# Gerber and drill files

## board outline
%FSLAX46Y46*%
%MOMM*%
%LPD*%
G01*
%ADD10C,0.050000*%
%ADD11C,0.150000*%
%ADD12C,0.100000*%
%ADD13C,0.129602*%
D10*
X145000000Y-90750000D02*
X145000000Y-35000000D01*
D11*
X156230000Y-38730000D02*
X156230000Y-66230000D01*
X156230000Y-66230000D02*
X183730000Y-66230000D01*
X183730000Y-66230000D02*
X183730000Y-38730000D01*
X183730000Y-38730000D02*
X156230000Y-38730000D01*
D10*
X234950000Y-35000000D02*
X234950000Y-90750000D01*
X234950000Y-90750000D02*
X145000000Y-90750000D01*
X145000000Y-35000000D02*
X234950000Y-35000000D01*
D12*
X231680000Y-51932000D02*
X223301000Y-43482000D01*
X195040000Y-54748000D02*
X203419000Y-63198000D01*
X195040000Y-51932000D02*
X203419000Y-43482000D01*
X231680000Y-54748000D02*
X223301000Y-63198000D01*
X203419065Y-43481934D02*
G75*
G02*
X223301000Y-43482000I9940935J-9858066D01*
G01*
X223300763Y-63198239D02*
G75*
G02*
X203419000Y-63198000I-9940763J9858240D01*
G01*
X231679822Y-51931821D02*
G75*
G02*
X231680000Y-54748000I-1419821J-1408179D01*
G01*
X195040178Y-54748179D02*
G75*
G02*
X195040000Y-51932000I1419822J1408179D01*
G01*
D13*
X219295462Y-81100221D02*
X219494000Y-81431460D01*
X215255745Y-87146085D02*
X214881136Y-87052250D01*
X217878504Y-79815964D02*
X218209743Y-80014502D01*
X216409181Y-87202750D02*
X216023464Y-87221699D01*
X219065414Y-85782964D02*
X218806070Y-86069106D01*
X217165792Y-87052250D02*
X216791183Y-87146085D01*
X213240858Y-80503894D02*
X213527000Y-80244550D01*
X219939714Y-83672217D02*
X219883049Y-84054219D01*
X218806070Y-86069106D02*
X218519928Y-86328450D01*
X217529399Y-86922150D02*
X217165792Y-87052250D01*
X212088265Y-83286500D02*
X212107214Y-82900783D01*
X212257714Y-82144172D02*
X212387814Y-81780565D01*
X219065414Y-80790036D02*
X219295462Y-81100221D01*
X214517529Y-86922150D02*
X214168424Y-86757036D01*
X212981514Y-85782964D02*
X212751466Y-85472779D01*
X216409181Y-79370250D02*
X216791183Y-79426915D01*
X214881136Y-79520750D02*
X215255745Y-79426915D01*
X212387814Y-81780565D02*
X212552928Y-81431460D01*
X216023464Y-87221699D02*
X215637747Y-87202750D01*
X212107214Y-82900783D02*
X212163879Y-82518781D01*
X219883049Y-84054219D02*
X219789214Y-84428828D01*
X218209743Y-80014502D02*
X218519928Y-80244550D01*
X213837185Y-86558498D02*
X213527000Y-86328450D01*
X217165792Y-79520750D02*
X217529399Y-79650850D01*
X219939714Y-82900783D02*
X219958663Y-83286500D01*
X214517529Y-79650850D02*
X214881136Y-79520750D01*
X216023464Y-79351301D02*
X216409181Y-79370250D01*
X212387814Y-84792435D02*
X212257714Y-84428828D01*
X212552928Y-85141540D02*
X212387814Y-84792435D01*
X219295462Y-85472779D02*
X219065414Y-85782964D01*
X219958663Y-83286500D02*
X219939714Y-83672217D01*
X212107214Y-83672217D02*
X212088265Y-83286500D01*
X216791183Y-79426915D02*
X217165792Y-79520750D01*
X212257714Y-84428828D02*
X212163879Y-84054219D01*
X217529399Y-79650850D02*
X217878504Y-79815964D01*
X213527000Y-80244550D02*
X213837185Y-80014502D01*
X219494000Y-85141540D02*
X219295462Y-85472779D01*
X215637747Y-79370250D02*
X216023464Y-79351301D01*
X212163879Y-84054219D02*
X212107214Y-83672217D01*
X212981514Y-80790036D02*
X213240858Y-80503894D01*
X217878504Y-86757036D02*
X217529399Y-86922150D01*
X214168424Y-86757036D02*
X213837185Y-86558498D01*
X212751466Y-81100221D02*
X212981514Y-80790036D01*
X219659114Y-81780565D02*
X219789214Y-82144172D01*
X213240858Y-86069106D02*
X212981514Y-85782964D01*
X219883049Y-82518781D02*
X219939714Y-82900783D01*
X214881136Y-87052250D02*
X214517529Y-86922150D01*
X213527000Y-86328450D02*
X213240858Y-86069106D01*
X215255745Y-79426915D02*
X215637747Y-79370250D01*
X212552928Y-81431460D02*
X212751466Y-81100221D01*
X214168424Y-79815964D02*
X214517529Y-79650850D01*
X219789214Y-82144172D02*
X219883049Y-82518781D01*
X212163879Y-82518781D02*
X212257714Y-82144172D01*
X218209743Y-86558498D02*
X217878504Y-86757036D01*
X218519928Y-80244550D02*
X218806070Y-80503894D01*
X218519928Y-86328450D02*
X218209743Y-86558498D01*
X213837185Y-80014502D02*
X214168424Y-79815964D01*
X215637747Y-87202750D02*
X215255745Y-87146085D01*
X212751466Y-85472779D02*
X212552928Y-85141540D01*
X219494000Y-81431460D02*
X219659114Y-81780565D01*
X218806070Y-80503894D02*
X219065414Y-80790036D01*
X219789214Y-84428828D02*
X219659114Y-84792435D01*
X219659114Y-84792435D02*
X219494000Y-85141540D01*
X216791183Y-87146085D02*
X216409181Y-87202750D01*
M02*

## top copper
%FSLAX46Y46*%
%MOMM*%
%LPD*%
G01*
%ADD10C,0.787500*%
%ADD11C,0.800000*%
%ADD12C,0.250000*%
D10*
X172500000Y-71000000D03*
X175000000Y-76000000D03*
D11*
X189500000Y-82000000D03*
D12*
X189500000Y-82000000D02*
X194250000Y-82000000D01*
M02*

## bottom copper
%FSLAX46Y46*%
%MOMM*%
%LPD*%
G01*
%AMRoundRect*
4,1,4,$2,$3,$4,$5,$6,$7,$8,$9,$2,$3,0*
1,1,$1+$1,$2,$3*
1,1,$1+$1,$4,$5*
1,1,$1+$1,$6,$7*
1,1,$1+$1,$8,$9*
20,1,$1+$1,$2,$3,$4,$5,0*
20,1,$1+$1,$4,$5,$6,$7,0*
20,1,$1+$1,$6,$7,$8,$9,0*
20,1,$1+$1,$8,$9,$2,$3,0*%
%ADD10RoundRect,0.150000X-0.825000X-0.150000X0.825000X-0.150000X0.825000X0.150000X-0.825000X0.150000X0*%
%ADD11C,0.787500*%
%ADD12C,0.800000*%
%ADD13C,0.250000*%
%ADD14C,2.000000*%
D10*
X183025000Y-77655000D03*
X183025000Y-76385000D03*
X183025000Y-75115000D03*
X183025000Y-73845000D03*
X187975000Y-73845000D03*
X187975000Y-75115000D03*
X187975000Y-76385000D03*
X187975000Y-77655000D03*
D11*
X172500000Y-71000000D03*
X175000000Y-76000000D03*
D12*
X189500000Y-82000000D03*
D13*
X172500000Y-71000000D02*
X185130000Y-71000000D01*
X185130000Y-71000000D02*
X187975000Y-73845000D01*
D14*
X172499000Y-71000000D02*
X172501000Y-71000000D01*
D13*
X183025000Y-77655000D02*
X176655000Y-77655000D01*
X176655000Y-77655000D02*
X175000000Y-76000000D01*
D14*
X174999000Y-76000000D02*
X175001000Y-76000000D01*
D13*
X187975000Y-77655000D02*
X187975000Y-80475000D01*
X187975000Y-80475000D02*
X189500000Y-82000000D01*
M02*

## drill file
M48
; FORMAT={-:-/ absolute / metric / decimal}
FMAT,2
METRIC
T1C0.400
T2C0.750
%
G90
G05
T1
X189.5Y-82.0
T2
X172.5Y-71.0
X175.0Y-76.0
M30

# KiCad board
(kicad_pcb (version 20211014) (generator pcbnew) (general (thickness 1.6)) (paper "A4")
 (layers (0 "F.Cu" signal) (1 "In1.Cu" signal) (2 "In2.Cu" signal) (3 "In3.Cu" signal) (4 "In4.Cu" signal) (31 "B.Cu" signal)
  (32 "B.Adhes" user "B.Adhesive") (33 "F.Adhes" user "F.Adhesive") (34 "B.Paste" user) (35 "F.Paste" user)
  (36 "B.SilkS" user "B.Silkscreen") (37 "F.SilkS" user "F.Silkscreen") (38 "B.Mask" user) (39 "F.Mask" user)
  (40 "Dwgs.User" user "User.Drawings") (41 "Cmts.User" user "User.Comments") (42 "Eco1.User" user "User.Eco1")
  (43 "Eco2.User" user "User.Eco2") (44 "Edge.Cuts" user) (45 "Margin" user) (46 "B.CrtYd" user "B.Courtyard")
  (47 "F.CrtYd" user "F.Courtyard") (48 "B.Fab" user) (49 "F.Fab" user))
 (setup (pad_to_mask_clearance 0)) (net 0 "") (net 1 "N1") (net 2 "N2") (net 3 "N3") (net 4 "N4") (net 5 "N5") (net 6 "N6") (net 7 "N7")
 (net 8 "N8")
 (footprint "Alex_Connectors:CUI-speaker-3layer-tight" (layer "F.Cu") (at 213.36 53.34 180)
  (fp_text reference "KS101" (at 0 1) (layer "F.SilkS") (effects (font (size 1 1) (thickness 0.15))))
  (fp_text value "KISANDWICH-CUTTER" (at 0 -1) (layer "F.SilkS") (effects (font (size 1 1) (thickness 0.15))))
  (fp_line (start -18.32 1.408) (end -9.941 9.858) (layer "Edge.Cuts") (width 0.1))
  (fp_line (start 18.32 -1.408) (end 9.941 -9.858) (layer "Edge.Cuts") (width 0.1))
  (fp_line (start 18.32 1.408) (end 9.941 9.858) (layer "Edge.Cuts") (width 0.1))
  (fp_line (start -18.32 -1.408) (end -9.941 -9.858) (layer "Edge.Cuts") (width 0.1))
  (fp_arc (start 9.940935 9.858066) (mid -0.000046 14.00013) (end -9.941 9.858) (layer "Edge.Cuts") (width 0.1))
  (fp_arc (start -9.940763 -9.858239) (mid 0.000168 -14.00013) (end 9.941 -9.858) (layer "Edge.Cuts") (width 0.1))
  (fp_arc (start -18.319822 1.408179) (mid -18.899716 0.000126) (end -18.32 -1.408) (layer "Edge.Cuts") (width 0.1))
  (fp_arc (start 18.319822 -1.408179) (mid 18.899716 -0.000126) (end 18.32 1.408) (layer "Edge.Cuts") (width 0.1)))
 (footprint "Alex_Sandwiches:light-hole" (layer "F.Cu") (at 201.93 77.47)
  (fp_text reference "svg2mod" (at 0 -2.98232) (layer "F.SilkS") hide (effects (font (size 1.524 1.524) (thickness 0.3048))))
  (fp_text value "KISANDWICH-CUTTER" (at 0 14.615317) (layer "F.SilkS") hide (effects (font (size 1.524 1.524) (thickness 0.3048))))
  (fp_line (start 17.365462 3.630221) (end 17.564 3.96146) (layer "Edge.Cuts") (width 0.129602))
  (fp_line (start 13.325745 9.676085) (end 12.951136 9.58225) (layer "Edge.Cuts") (width 0.129602))
  (fp_line (start 15.948504 2.345964) (end 16.279743 2.544502) (layer "Edge.Cuts") (width 0.129602))
  (fp_line (start 14.479181 9.73275) (end 14.093464 9.751699) (layer "Edge.Cuts") (width 0.129602))
  (fp_line (start 17.135414 8.312964) (end 16.87607 8.599106) (layer "Edge.Cuts") (width 0.129602))
  (fp_line (start 15.235792 9.58225) (end 14.861183 9.676085) (layer "Edge.Cuts") (width 0.129602))
  (fp_line (start 11.310858 3.033894) (end 11.597 2.77455) (layer "Edge.Cuts") (width 0.129602))
  (fp_line (start 18.009714 6.202217) (end 17.953049 6.584219) (layer "Edge.Cuts") (width 0.129602))
  (fp_line (start 16.87607 8.599106) (end 16.589928 8.85845) (layer "Edge.Cuts") (width 0.129602))
  (fp_line (start 15.599399 9.45215) (end 15.235792 9.58225) (layer "Edge.Cuts") (width 0.129602))
  (fp_line (start 10.158265 5.8165) (end 10.177214 5.430783) (layer "Edge.Cuts") (width 0.129602))
  (fp_line (start 10.327714 4.674172) (end 10.457814 4.310565) (layer "Edge.Cuts") (width 0.129602))
  (fp_line (start 17.135414 3.320036) (end 17.365462 3.630221) (layer "Edge.Cuts") (width 0.129602))
  (fp_line (start 12.587529 9.45215) (end 12.238424 9.287036) (layer "Edge.Cuts") (width 0.129602))
  (fp_line (start 11.051514 8.312964) (end 10.821466 8.002779) (layer "Edge.Cuts") (width 0.129602))
  (fp_line (start 14.479181 1.90025) (end 14.861183 1.956915) (layer "Edge.Cuts") (width 0.129602))
  (fp_line (start 12.951136 2.05075) (end 13.325745 1.956915) (layer "Edge.Cuts") (width 0.129602))
  (fp_line (start 10.457814 4.310565) (end 10.622928 3.96146) (layer "Edge.Cuts") (width 0.129602))
  (fp_line (start 14.093464 9.751699) (end 13.707747 9.73275) (layer "Edge.Cuts") (width 0.129602))
  (fp_line (start 10.177214 5.430783) (end 10.233879 5.048781) (layer "Edge.Cuts") (width 0.129602))
  (fp_line (start 17.953049 6.584219) (end 17.859214 6.958828) (layer "Edge.Cuts") (width 0.129602))
  (fp_line (start 16.279743 2.544502) (end 16.589928 2.77455) (layer "Edge.Cuts") (width 0.129602))
  (fp_line (start 11.907185 9.088498) (end 11.597 8.85845) (layer "Edge.Cuts") (width 0.129602))
  (fp_line (start 15.235792 2.05075) (end 15.599399 2.18085) (layer "Edge.Cuts") (width 0.129602))
  (fp_line (start 18.009714 5.430783) (end 18.028663 5.8165) (layer "Edge.Cuts") (width 0.129602))
  (fp_line (start 12.587529 2.18085) (end 12.951136 2.05075) (layer "Edge.Cuts") (width 0.129602))
  (fp_line (start 14.093464 1.881301) (end 14.479181 1.90025) (layer "Edge.Cuts") (width 0.129602))
  (fp_line (start 10.457814 7.322435) (end 10.327714 6.958828) (layer "Edge.Cuts") (width 0.129602))
  (fp_line (start 10.622928 7.67154) (end 10.457814 7.322435) (layer "Edge.Cuts") (width 0.129602))
  (fp_line (start 17.365462 8.002779) (end 17.135414 8.312964) (layer "Edge.Cuts") (width 0.129602))
  (fp_line (start 18.028663 5.8165) (end 18.009714 6.202217) (layer "Edge.Cuts") (width 0.129602))
  (fp_line (start 10.177214 6.202217) (end 10.158265 5.8165) (layer "Edge.Cuts") (width 0.129602))
  (fp_line (start 14.861183 1.956915) (end 15.235792 2.05075) (layer "Edge.Cuts") (width 0.129602))
  (fp_line (start 10.327714 6.958828) (end 10.233879 6.584219) (layer "Edge.Cuts") (width 0.129602))
  (fp_line (start 15.599399 2.18085) (end 15.948504 2.345964) (layer "Edge.Cuts") (width 0.129602))
  (fp_line (start 11.597 2.77455) (end 11.907185 2.544502) (layer "Edge.Cuts") (width 0.129602))
  (fp_line (start 17.564 7.67154) (end 17.365462 8.002779) (layer "Edge.Cuts") (width 0.129602))
  (fp_line (start 13.707747 1.90025) (end 14.093464 1.881301) (layer "Edge.Cuts") (width 0.129602))
  (fp_line (start 10.233879 6.584219) (end 10.177214 6.202217) (layer "Edge.Cuts") (width 0.129602))
  (fp_line (start 11.051514 3.320036) (end 11.310858 3.033894) (layer "Edge.Cuts") (width 0.129602))
  (fp_line (start 15.948504 9.287036) (end 15.599399 9.45215) (layer "Edge.Cuts") (width 0.129602))
  (fp_line (start 12.238424 9.287036) (end 11.907185 9.088498) (layer "Edge.Cuts") (width 0.129602))
  (fp_line (start 10.821466 3.630221) (end 11.051514 3.320036) (layer "Edge.Cuts") (width 0.129602))
  (fp_line (start 17.729114 4.310565) (end 17.859214 4.674172) (layer "Edge.Cuts") (width 0.129602))
  (fp_line (start 11.310858 8.599106) (end 11.051514 8.312964) (layer "Edge.Cuts") (width 0.129602))
  (fp_line (start 17.953049 5.048781) (end 18.009714 5.430783) (layer "Edge.Cuts") (width 0.129602))
  (fp_line (start 12.951136 9.58225) (end 12.587529 9.45215) (layer "Edge.Cuts") (width 0.129602))
  (fp_line (start 11.597 8.85845) (end 11.310858 8.599106) (layer "Edge.Cuts") (width 0.129602))
  (fp_line (start 13.325745 1.956915) (end 13.707747 1.90025) (layer "Edge.Cuts") (width 0.129602))
  (fp_line (start 10.622928 3.96146) (end 10.821466 3.630221) (layer "Edge.Cuts") (width 0.129602))
  (fp_line (start 12.238424 2.345964) (end 12.587529 2.18085) (layer "Edge.Cuts") (width 0.129602))
  (fp_line (start 17.859214 4.674172) (end 17.953049 5.048781) (layer "Edge.Cuts") (width 0.129602))
  (fp_line (start 10.233879 5.048781) (end 10.327714 4.674172) (layer "Edge.Cuts") (width 0.129602))
  (fp_line (start 16.279743 9.088498) (end 15.948504 9.287036) (layer "Edge.Cuts") (width 0.129602))
  (fp_line (start 16.589928 2.77455) (end 16.87607 3.033894) (layer "Edge.Cuts") (width 0.129602))
  (fp_line (start 16.589928 8.85845) (end 16.279743 9.088498) (layer "Edge.Cuts") (width 0.129602))
  (fp_line (start 11.907185 2.544502) (end 12.238424 2.345964) (layer "Edge.Cuts") (width 0.129602))
  (fp_line (start 13.707747 9.73275) (end 13.325745 9.676085) (layer "Edge.Cuts") (width 0.129602))
  (fp_line (start 10.821466 8.002779) (end 10.622928 7.67154) (layer "Edge.Cuts") (width 0.129602))
  (fp_line (start 17.564 3.96146) (end 17.729114 4.310565) (layer "Edge.Cuts") (width 0.129602))
  (fp_line (start 16.87607 3.033894) (end 17.135414 3.320036) (layer "Edge.Cuts") (width 0.129602))
  (fp_line (start 17.859214 6.958828) (end 17.729114 7.322435) (layer "Edge.Cuts") (width 0.129602))
  (fp_line (start 17.729114 7.322435) (end 17.564 7.67154) (layer "Edge.Cuts") (width 0.129602))
  (fp_line (start 14.861183 9.676085) (end 14.479181 9.73275) (layer "Edge.Cuts") (width 0.129602)))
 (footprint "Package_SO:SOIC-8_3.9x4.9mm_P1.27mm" (layer "B.Cu") (at 185.5 75.75)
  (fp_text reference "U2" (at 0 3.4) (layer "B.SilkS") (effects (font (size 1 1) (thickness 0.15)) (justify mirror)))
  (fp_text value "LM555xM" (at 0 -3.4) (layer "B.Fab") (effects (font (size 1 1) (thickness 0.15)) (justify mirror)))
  (pad "1" smd roundrect locked (at -2.475 1.905) (size 1.95 0.6) (layers "B.Cu" "B.Paste" "B.Mask") (roundrect_rratio 0.25) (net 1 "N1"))
  (pad "2" smd roundrect locked (at -2.475 0.635) (size 1.95 0.6) (layers "B.Cu" "B.Paste" "B.Mask") (roundrect_rratio 0.25) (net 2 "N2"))
  (pad "3" smd roundrect locked (at -2.475 -0.635) (size 1.95 0.6) (layers "B.Cu" "B.Paste" "B.Mask") (roundrect_rratio 0.25) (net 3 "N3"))
  (pad "4" smd roundrect locked (at -2.475 -1.905) (size 1.95 0.6) (layers "B.Cu" "B.Paste" "B.Mask") (roundrect_rratio 0.25) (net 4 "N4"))
  (pad "5" smd roundrect locked (at 2.475 -1.905) (size 1.95 0.6) (layers "B.Cu" "B.Paste" "B.Mask") (roundrect_rratio 0.25) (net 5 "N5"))
  (pad "6" smd roundrect locked (at 2.475 -0.635) (size 1.95 0.6) (layers "B.Cu" "B.Paste" "B.Mask") (roundrect_rratio 0.25) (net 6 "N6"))
  (pad "7" smd roundrect locked (at 2.475 0.635) (size 1.95 0.6) (layers "B.Cu" "B.Paste" "B.Mask") (roundrect_rratio 0.25) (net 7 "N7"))
  (pad "8" smd roundrect locked (at 2.475 1.905) (size 1.95 0.6) (layers "B.Cu" "B.Paste" "B.Mask") (roundrect_rratio 0.25) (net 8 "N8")))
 (gr_line (start 145 90.75) (end 145 35) (layer "Edge.Cuts") (width 0.05))
 (gr_line (start 156.23 38.73) (end 156.23 66.23) (layer "Edge.Cuts") (width 0.15))
 (gr_line (start 156.23 66.23) (end 183.73 66.23) (layer "Edge.Cuts") (width 0.15))
 (gr_line (start 183.73 66.23) (end 183.73 38.73) (layer "Edge.Cuts") (width 0.15))
 (gr_line (start 183.73 38.73) (end 156.23 38.73) (layer "Edge.Cuts") (width 0.15))
 (gr_line (start 234.95 35) (end 234.95 90.75) (layer "Edge.Cuts") (width 0.05))
 (gr_line (start 234.95 90.75) (end 145 90.75) (layer "Edge.Cuts") (width 0.05))
 (gr_line (start 145 35) (end 234.95 35) (layer "Edge.Cuts") (width 0.05))
 (via (at 172.5 71) (size 0.7875) (drill 0.75) (layers "F.Cu" "B.Cu") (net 5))
 (segment (start 172.5 71) (end 185.13 71) (width 0.25) (layer "B.Cu") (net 5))
 (segment (start 185.13 71) (end 187.975 73.845) (width 0.25) (layer "B.Cu") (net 5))
 (segment (start 172.499 71) (end 172.501 71) (width 2) (layer "B.Cu") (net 5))
 (via (at 175 76) (size 0.7875) (drill 0.75) (layers "F.Cu" "B.Cu") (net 1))
 (segment (start 183.025 77.655) (end 176.655 77.655) (width 0.25) (layer "B.Cu") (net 1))
 (segment (start 176.655 77.655) (end 175 76) (width 0.25) (layer "B.Cu") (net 1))
 (segment (start 174.999 76) (end 175.001 76) (width 2) (layer "B.Cu") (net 1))
 (segment (start 189.5 82) (end 194.25 82) (width 0.25) (layer "F.Cu") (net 8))
 (segment (start 187.975 77.655) (end 187.975 80.475) (width 0.25) (layer "B.Cu") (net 8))
 (segment (start 187.975 80.475) (end 189.5 82) (width 0.25) (layer "B.Cu") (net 8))
 (via (at 189.5 82) (size 0.8) (drill 0.4) (layers "F.Cu" "B.Cu") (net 8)))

